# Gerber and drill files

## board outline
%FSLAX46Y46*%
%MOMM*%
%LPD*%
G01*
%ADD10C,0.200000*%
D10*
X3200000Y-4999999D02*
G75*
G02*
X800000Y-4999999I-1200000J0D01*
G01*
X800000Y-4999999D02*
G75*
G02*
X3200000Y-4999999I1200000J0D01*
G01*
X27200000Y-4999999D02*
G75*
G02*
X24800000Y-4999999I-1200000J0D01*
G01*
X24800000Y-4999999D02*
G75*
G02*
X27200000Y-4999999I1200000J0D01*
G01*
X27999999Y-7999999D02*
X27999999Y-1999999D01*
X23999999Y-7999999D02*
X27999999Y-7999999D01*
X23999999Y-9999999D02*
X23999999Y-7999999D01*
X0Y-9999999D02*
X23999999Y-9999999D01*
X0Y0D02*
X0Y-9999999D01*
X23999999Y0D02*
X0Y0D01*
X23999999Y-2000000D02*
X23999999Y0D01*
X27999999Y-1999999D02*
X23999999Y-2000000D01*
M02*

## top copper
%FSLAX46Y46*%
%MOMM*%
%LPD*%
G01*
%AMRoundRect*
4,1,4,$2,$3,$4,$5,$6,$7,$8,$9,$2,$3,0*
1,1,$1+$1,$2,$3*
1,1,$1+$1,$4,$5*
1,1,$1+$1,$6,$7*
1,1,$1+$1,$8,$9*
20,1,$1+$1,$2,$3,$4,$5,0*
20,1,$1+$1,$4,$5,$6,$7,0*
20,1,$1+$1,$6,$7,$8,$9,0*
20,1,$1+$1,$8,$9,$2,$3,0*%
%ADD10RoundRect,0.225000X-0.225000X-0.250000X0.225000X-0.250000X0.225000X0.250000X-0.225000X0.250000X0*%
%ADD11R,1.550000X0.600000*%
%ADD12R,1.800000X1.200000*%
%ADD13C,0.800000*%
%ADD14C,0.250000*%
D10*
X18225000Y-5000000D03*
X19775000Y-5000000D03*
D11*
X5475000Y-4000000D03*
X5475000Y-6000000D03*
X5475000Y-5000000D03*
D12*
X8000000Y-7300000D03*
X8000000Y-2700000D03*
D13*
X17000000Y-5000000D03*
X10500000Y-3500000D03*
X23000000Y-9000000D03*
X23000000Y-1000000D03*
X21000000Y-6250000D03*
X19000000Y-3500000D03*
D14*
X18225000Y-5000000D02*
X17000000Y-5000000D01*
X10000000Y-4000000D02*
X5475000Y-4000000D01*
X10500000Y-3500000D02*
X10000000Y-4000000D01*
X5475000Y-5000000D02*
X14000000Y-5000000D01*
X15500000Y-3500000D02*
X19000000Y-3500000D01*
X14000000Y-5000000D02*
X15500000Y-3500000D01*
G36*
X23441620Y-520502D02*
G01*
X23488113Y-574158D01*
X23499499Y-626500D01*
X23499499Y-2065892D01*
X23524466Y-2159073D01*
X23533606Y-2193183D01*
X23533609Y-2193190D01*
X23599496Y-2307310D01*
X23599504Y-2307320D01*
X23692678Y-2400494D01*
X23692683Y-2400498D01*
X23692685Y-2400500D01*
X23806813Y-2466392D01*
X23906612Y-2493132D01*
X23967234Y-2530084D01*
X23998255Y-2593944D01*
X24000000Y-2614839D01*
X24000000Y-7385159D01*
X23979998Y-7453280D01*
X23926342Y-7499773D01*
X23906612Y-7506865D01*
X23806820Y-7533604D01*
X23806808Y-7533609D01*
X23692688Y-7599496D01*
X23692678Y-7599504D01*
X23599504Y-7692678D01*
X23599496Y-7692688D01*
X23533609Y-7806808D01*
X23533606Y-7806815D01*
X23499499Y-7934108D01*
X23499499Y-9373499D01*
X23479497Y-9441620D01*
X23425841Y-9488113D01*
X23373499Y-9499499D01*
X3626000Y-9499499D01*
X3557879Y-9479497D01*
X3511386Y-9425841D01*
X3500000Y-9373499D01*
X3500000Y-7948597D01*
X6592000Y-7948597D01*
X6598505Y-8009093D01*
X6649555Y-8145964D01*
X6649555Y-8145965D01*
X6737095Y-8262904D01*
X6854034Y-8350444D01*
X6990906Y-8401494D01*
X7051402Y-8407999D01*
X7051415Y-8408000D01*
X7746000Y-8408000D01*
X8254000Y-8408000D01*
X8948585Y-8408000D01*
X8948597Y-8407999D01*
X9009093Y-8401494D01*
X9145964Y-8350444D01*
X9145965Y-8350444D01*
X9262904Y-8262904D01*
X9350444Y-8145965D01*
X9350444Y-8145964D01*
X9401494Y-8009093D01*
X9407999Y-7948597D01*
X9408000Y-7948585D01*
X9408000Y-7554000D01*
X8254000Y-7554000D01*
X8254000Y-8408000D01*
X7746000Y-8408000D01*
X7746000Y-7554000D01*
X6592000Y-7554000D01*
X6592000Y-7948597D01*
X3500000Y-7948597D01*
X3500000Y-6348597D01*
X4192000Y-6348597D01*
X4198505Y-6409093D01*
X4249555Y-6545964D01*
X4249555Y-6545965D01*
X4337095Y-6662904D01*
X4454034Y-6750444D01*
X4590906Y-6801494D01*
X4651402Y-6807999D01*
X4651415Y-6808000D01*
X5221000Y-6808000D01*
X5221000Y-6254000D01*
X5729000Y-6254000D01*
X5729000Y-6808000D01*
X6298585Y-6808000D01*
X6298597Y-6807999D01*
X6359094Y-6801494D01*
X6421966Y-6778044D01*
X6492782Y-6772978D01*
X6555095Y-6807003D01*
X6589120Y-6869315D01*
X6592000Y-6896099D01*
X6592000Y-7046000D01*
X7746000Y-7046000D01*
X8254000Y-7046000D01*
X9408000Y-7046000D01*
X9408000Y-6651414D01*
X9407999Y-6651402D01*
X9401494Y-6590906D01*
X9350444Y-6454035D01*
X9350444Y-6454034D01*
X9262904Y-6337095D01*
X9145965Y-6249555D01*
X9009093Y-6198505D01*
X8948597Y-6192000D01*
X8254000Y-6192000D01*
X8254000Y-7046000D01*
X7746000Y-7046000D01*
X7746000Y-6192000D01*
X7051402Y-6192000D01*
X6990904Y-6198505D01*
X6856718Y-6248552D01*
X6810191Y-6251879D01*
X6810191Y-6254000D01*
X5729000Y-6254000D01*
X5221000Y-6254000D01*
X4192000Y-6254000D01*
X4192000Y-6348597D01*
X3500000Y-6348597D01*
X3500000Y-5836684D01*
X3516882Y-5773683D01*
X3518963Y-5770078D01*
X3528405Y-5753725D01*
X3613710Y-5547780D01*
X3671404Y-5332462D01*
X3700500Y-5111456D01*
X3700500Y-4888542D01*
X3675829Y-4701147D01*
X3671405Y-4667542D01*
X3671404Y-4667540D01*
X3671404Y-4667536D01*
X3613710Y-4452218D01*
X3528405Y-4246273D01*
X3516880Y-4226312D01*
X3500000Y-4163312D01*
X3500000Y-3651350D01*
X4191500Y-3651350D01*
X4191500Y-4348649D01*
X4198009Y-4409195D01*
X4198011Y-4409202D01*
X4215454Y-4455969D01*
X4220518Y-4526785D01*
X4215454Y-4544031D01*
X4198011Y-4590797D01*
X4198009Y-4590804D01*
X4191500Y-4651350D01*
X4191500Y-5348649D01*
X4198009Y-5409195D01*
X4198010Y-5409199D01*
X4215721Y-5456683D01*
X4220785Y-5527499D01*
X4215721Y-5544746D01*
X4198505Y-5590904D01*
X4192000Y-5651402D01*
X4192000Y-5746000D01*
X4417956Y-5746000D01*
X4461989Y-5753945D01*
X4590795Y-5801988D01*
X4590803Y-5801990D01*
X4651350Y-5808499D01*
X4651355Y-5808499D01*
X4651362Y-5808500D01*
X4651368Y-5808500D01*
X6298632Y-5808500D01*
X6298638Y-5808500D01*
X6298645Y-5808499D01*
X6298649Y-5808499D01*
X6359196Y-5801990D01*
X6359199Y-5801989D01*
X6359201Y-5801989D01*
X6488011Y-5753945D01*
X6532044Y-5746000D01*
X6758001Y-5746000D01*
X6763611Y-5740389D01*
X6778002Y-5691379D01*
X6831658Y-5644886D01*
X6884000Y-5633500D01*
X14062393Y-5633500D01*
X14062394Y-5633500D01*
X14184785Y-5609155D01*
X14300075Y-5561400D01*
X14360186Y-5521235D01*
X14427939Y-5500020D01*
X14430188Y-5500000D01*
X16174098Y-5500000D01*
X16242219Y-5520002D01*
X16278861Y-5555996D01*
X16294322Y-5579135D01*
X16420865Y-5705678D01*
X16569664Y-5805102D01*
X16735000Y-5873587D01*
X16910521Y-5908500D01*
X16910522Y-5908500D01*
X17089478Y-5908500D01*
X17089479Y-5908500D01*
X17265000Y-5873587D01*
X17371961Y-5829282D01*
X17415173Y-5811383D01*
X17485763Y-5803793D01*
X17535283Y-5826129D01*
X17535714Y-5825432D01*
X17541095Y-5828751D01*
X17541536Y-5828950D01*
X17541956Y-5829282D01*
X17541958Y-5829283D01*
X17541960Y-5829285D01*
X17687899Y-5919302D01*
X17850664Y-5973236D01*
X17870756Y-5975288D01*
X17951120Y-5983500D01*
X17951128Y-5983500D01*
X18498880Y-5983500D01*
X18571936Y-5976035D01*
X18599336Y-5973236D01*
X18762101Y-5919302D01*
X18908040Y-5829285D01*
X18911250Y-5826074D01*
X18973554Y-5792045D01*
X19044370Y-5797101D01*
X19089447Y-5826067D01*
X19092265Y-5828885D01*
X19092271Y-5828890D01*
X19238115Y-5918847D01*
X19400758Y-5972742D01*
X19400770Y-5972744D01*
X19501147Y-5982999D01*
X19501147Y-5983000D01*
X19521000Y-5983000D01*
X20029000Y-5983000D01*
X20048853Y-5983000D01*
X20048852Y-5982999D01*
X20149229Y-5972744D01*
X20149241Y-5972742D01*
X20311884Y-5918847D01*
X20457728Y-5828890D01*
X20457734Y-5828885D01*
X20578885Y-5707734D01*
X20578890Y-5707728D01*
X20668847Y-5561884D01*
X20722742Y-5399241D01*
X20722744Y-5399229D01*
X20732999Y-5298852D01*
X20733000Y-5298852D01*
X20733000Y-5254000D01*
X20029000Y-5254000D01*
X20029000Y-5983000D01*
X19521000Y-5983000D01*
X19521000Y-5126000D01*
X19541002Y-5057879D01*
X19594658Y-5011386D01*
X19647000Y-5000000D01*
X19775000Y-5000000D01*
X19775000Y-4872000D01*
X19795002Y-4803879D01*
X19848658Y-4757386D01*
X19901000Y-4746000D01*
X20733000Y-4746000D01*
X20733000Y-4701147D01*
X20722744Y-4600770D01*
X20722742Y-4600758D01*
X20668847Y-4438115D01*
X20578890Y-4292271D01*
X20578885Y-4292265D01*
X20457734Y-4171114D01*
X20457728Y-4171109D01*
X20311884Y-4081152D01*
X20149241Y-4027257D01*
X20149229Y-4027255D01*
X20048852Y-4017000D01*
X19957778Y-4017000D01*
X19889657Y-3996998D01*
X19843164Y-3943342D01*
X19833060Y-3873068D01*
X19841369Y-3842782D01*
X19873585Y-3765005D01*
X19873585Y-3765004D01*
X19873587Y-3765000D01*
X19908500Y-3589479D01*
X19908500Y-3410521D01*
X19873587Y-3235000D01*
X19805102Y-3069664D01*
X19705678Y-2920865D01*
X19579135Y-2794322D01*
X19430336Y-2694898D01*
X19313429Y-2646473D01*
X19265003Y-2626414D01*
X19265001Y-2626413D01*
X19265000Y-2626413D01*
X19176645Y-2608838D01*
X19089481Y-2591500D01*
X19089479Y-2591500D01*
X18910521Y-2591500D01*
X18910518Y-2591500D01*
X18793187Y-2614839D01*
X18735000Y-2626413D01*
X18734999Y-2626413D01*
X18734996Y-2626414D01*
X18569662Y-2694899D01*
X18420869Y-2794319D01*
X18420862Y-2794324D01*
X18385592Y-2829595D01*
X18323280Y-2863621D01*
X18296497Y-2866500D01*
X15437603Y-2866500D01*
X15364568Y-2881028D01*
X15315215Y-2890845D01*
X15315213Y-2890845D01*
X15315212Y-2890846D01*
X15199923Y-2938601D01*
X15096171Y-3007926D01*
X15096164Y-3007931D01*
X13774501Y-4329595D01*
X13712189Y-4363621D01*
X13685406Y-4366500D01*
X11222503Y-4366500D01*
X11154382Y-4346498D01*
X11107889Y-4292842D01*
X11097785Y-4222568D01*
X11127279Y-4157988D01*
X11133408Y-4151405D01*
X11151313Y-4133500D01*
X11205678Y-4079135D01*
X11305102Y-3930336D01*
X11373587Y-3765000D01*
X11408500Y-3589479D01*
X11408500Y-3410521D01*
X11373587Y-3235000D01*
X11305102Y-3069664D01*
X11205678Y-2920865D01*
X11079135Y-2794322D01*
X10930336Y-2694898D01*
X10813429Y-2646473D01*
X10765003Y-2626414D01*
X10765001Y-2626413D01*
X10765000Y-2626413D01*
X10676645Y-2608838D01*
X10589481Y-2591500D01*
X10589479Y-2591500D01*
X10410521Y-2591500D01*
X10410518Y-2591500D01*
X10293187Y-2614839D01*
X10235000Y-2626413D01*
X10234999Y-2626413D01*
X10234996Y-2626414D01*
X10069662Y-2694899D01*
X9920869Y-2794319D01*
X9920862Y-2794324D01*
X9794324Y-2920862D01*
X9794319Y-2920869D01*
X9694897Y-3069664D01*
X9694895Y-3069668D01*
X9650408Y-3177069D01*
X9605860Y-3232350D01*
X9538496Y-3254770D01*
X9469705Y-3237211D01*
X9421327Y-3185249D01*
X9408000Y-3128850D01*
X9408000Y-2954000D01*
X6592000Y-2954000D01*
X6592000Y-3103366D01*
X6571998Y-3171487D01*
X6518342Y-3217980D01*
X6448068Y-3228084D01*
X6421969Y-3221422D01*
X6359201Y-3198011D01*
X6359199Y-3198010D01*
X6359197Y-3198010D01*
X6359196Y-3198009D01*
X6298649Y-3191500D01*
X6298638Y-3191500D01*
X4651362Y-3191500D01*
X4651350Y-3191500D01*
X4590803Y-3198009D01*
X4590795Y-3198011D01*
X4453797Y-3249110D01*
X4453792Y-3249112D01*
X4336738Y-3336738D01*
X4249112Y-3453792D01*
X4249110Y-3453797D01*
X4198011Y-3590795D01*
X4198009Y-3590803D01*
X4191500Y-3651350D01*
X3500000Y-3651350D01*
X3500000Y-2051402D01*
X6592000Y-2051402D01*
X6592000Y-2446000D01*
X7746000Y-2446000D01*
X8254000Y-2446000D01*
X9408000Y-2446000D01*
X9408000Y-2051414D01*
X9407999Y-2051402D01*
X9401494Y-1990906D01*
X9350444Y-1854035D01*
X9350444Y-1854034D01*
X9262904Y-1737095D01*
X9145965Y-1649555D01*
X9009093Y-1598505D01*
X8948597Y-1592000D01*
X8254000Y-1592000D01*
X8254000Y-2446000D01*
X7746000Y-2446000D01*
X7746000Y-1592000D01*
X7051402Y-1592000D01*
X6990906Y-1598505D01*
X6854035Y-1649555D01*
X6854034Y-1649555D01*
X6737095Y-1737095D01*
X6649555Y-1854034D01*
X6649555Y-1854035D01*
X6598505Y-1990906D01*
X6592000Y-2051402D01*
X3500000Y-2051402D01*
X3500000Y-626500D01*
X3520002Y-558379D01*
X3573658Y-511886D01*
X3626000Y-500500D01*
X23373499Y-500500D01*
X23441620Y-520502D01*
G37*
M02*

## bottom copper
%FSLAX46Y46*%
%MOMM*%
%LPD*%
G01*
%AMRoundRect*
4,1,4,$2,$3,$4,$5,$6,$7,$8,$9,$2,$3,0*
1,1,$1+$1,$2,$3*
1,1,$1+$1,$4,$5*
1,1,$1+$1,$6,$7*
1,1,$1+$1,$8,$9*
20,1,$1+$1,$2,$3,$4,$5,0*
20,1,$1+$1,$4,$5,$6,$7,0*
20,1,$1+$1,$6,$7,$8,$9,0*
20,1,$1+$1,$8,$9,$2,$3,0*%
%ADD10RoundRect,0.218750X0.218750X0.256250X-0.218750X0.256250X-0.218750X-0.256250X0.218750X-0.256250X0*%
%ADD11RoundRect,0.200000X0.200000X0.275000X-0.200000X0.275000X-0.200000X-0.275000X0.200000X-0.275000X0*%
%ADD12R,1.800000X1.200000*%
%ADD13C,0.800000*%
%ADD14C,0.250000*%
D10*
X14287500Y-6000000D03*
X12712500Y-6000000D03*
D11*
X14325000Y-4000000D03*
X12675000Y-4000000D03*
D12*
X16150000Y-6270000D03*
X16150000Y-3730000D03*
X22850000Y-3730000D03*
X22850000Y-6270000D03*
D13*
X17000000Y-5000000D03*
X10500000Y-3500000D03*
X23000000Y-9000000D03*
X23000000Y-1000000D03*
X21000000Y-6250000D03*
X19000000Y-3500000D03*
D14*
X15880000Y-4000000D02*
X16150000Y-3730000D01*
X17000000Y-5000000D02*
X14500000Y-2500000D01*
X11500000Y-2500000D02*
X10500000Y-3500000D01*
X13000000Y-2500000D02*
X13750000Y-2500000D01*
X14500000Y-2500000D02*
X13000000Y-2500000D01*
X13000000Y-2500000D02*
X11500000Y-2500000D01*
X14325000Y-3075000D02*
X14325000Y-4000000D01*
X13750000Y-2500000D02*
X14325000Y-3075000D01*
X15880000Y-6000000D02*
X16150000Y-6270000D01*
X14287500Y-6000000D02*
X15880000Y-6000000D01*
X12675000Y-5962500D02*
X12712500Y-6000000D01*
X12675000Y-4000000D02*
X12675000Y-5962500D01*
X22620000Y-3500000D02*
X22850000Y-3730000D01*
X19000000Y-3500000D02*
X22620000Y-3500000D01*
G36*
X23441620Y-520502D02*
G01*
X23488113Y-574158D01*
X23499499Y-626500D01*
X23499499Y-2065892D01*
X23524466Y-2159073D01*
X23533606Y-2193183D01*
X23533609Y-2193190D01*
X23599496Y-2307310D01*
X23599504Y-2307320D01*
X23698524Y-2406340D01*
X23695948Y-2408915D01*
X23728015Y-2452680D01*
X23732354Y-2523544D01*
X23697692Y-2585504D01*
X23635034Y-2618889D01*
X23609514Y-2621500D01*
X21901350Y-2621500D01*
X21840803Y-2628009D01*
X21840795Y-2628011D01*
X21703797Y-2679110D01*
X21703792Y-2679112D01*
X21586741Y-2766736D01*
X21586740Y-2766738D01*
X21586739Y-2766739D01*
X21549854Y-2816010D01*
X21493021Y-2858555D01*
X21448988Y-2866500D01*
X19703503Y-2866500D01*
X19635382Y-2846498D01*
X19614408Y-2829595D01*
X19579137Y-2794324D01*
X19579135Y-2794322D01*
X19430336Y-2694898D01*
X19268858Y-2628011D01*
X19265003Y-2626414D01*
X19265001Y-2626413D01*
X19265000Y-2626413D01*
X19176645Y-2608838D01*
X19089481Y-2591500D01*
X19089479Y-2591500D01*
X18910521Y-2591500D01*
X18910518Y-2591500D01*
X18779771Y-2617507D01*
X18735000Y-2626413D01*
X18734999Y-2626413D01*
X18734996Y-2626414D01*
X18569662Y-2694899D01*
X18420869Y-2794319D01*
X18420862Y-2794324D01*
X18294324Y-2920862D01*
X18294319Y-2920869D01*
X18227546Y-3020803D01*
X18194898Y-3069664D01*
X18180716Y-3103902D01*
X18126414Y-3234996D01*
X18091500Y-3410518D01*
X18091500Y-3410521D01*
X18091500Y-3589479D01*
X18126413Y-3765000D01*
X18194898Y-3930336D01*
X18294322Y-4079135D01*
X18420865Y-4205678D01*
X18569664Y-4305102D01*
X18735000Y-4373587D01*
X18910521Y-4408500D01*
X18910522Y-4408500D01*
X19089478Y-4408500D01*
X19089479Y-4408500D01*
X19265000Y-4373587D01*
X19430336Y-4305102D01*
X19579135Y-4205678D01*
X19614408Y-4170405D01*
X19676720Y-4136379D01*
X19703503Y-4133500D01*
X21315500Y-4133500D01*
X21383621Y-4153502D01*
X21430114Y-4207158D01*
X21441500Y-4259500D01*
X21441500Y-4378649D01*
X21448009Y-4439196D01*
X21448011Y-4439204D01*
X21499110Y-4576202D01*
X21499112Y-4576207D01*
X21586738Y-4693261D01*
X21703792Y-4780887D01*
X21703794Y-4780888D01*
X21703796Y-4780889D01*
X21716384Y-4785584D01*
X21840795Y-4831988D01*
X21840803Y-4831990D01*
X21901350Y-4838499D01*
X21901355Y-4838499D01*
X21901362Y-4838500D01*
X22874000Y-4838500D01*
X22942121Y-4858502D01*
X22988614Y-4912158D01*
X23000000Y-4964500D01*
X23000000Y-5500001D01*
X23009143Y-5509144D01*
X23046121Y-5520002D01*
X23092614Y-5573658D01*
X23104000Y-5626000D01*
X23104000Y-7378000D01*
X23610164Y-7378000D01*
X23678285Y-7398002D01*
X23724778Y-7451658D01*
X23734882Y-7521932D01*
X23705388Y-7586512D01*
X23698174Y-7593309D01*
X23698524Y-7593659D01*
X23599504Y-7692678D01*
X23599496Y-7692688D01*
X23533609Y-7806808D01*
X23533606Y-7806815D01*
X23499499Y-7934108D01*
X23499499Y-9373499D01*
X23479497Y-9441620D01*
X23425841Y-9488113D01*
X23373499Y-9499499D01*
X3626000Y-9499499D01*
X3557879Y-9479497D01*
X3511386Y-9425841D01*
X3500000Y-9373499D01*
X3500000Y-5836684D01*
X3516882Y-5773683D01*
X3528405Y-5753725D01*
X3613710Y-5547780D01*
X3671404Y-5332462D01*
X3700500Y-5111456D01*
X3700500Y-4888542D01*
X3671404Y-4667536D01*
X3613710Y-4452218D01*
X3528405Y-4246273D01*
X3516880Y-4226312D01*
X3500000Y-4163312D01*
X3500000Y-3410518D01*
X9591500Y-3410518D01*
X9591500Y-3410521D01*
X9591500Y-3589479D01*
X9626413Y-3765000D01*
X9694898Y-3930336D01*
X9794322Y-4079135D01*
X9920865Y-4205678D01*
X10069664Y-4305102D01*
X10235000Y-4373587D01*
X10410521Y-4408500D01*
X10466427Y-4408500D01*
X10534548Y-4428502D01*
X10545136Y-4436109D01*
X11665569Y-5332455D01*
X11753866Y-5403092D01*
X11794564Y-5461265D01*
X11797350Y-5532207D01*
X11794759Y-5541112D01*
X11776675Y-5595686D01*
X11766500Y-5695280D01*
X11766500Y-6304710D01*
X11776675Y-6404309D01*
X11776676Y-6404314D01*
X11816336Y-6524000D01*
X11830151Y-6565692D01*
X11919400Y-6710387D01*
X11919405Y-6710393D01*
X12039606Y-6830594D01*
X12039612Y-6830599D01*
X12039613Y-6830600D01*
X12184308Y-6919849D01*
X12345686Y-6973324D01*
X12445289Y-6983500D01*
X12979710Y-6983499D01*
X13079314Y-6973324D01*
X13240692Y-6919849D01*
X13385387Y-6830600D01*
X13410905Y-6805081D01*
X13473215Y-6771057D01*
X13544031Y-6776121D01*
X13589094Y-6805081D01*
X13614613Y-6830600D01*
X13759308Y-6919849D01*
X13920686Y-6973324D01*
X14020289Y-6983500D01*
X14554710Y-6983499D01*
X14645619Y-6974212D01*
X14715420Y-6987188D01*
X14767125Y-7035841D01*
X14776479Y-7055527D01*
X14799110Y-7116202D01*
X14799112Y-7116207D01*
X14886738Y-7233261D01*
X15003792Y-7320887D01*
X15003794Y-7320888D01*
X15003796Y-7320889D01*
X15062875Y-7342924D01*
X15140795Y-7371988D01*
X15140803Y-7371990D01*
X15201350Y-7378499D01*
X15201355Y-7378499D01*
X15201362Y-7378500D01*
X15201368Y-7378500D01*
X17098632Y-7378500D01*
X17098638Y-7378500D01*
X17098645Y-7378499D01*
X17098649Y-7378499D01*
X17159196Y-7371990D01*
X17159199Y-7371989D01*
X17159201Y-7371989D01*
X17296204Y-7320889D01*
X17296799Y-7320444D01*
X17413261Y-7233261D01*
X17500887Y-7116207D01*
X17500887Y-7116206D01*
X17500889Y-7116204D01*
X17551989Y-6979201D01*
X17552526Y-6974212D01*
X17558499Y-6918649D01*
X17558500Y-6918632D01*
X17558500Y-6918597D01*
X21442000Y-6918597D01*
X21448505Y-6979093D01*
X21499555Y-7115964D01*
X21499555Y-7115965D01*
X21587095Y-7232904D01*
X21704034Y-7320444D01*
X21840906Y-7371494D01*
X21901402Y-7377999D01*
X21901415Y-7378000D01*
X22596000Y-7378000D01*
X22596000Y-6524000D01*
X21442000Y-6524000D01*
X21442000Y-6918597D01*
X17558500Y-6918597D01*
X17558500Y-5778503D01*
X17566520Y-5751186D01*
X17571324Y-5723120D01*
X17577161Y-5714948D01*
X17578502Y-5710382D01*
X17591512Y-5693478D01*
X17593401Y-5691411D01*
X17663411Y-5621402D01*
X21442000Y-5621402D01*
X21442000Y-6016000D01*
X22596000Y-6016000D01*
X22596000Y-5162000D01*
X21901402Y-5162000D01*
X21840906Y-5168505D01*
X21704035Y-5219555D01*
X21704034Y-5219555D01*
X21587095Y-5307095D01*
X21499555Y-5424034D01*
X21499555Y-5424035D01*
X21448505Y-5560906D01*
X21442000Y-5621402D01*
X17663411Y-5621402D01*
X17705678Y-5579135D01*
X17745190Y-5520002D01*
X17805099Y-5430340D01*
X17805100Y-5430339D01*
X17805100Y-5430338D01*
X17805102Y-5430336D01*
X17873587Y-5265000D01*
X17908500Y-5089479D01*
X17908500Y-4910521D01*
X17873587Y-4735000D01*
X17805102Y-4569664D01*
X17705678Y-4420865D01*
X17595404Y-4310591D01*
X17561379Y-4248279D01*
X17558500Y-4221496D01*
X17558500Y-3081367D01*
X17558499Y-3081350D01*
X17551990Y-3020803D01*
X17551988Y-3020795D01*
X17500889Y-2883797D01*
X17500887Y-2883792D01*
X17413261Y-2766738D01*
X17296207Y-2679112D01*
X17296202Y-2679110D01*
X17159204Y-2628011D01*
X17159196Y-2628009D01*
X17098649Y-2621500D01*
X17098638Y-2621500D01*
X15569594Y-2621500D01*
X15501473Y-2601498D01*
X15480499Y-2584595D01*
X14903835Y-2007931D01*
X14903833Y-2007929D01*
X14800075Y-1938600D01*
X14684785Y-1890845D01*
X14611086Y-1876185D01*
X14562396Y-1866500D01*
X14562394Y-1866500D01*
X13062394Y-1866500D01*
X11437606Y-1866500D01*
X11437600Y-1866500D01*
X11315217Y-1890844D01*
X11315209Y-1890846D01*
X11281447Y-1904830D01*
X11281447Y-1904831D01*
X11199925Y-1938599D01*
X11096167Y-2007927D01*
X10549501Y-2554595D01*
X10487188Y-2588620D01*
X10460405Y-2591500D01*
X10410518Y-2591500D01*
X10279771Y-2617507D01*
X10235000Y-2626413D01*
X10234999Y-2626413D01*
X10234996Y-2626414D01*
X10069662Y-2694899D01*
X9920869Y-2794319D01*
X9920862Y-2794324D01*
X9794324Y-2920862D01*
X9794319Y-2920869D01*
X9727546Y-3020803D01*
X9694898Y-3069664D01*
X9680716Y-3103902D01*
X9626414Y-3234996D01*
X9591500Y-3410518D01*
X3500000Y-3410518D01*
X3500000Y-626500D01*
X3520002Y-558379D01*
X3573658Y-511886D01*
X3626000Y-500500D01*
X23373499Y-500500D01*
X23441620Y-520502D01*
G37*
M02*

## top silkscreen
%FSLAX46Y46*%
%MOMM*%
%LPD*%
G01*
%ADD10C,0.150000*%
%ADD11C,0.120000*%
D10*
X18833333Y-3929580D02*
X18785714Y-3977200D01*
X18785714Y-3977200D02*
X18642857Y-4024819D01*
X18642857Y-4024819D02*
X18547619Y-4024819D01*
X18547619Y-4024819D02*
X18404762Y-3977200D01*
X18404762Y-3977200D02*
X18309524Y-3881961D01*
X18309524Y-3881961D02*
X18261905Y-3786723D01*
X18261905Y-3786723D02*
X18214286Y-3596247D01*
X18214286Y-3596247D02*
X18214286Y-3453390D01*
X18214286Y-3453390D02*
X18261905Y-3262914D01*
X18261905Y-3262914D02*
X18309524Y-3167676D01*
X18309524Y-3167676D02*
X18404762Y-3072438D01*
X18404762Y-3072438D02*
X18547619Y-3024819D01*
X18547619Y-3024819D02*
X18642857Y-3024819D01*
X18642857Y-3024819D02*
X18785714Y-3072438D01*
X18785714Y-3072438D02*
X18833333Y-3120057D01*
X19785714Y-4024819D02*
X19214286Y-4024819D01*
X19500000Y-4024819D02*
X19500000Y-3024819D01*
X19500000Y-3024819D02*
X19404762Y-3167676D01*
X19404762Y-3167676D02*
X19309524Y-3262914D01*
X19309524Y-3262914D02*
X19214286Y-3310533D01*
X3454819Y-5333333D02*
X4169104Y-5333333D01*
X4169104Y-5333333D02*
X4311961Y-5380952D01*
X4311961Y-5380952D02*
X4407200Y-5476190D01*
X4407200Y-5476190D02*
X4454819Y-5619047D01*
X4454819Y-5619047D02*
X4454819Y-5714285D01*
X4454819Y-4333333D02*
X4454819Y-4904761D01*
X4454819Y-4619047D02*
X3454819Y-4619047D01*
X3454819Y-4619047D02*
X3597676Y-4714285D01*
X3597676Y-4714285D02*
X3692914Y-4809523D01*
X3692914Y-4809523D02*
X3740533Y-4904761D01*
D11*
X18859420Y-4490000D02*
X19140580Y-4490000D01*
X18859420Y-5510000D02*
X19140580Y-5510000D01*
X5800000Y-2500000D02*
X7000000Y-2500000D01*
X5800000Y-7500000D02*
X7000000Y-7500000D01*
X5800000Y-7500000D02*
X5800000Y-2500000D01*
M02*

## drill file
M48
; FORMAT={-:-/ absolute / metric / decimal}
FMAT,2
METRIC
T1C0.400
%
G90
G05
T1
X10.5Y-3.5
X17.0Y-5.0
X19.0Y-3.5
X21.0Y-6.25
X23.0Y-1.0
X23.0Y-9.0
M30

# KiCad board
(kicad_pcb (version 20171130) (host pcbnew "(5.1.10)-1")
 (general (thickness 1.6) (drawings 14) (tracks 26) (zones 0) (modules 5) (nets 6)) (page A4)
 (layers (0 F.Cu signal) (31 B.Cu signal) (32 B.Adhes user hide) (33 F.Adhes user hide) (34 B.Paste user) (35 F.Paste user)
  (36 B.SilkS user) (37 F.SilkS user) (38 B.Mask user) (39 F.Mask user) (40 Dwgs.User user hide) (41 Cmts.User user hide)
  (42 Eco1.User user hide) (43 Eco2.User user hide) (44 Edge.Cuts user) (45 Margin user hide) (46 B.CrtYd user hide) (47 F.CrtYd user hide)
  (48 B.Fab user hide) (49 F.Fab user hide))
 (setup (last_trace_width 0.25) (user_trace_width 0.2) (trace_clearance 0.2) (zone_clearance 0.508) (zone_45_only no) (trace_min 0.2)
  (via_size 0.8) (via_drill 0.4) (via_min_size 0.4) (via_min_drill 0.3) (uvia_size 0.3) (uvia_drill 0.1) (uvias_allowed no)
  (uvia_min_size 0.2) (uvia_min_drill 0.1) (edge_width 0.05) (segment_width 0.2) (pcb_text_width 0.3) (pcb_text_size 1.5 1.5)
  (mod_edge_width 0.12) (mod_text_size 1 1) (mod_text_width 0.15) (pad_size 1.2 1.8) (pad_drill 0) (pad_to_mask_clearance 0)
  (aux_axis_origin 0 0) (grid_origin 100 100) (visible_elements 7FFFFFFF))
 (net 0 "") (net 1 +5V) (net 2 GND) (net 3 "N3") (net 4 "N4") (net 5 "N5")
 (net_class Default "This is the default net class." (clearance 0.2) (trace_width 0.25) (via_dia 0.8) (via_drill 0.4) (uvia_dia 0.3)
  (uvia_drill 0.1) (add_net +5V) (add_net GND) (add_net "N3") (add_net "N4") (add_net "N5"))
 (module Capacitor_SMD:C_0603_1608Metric (layer F.Cu) (at 19 5)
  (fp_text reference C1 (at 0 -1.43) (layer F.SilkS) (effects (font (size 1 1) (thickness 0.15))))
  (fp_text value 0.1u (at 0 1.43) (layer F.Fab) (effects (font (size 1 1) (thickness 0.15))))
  (fp_line (start -0.14058 -0.51) (end 0.14058 -0.51) (layer F.SilkS) (width 0.12))
  (fp_line (start -0.14058 0.51) (end 0.14058 0.51) (layer F.SilkS) (width 0.12))
  (pad 1 smd roundrect (at -0.775 0) (size 0.9 0.95) (layers F.Cu F.Paste F.Mask) (roundrect_rratio 0.25) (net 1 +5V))
  (pad 2 smd roundrect (at 0.775 0) (size 0.9 0.95) (layers F.Cu F.Paste F.Mask) (roundrect_rratio 0.25) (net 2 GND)))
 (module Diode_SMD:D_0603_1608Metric (layer B.Cu) (at 13.5 6 180)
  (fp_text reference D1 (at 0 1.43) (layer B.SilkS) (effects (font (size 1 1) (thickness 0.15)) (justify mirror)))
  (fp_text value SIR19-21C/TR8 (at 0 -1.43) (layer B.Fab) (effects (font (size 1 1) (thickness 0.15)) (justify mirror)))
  (pad 1 smd roundrect (at -0.7875 0 180) (size 0.875 0.95) (layers B.Cu B.Paste B.Mask) (roundrect_rratio 0.25) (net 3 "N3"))
  (pad 2 smd roundrect (at 0.7875 0 180) (size 0.875 0.95) (layers B.Cu B.Paste B.Mask) (roundrect_rratio 0.25) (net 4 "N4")))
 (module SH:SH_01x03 (layer F.Cu) (at 8 5 90)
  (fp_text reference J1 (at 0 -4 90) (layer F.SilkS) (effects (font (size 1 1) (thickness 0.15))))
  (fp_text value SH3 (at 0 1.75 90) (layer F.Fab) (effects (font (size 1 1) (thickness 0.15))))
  (fp_line (start 2.5 -2.2) (end 2.5 -1) (layer F.SilkS) (width 0.12))
  (fp_line (start -2.5 -2.2) (end -2.5 -1) (layer F.SilkS) (width 0.12))
  (fp_line (start -2.5 -2.2) (end 2.5 -2.2) (layer F.SilkS) (width 0.12))
  (pad 3 smd rect (at 1 -2.525 90) (size 0.6 1.55) (layers F.Cu F.Paste F.Mask) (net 1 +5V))
  (pad 1 smd rect (at -1 -2.525 90) (size 0.6 1.55) (layers F.Cu F.Paste F.Mask) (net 2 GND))
  (pad 2 smd rect (at 0 -2.525 90) (size 0.6 1.55) (layers F.Cu F.Paste F.Mask) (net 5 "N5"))
  (pad MP smd rect (at -2.3 0 90) (size 1.2 1.8) (layers F.Cu F.Paste F.Mask) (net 2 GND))
  (pad MP smd rect (at 2.3 0 90) (size 1.2 1.8) (layers F.Cu F.Paste F.Mask) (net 2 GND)))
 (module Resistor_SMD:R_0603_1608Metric (layer B.Cu) (at 13.5 4 180)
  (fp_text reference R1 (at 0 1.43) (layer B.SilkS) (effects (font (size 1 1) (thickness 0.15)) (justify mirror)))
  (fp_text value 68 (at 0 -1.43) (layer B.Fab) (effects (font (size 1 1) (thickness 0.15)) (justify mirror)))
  (pad 1 smd roundrect (at -0.825 0 180) (size 0.8 0.95) (layers B.Cu B.Paste B.Mask) (roundrect_rratio 0.25) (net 1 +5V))
  (pad 2 smd roundrect (at 0.825 0 180) (size 0.8 0.95) (layers B.Cu B.Paste B.Mask) (roundrect_rratio 0.25) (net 4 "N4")))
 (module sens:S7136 (layer B.Cu) (at 19.5 5)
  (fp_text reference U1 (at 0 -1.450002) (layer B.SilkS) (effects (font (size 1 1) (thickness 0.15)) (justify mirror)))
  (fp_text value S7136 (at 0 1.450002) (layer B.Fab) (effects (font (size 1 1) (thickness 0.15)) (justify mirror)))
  (pad 1 smd rect (at -3.35 1.27) (size 1.8 1.2) (layers B.Cu B.Paste B.Mask) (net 3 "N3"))
  (pad 2 smd rect (at -3.35 -1.27) (size 1.8 1.2) (layers B.Cu B.Paste B.Mask) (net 1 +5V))
  (pad 3 smd rect (at 3.35 -1.27) (size 1.8 1.2) (layers B.Cu B.Paste B.Mask) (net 5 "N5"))
  (pad 4 smd rect (at 3.35 1.27) (size 1.8 1.2) (layers B.Cu B.Paste B.Mask) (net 2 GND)))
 (gr_circle (center 2 4.999999) (end 3.2 4.999999) (layer Edge.Cuts) (width 0.2))
 (gr_circle (center 26 4.999999) (end 27.2 4.999999) (layer Edge.Cuts) (width 0.2))
 (gr_line (start 27.999999 7.999999) (end 27.999999 1.999999) (layer Edge.Cuts) (width 0.2))
 (gr_line (start 23.999999 7.999999) (end 27.999999 7.999999) (layer Edge.Cuts) (width 0.2))
 (gr_line (start 23.999999 9.999999) (end 23.999999 7.999999) (layer Edge.Cuts) (width 0.2))
 (gr_line (start 0 9.999999) (end 23.999999 9.999999) (layer Edge.Cuts) (width 0.2))
 (gr_line (start 0 0) (end 0 9.999999) (layer Edge.Cuts) (width 0.2))
 (gr_line (start 23.999999 0) (end 0 0) (layer Edge.Cuts) (width 0.2))
 (gr_line (start 23.999999 2) (end 23.999999 0) (layer Edge.Cuts) (width 0.2))
 (gr_line (start 27.999999 1.999999) (end 23.999999 2) (layer Edge.Cuts) (width 0.2))
 (segment (start 15.88 4) (end 16.15 3.73) (width 0.25) (layer B.Cu) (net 1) (status 30))
 (via (at 17 5) (size 0.8) (drill 0.4) (layers F.Cu B.Cu) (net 1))
 (segment (start 18.225 5) (end 17 5) (width 0.25) (layer F.Cu) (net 1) (status 10))
 (segment (start 17 5) (end 14.5 2.5) (width 0.25) (layer B.Cu) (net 1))
 (via (at 10.5 3.5) (size 0.8) (drill 0.4) (layers F.Cu B.Cu) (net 1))
 (segment (start 11.5 2.5) (end 10.5 3.5) (width 0.25) (layer B.Cu) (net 1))
 (segment (start 10 4) (end 5.475 4) (width 0.25) (layer F.Cu) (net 1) (status 20))
 (segment (start 10.5 3.5) (end 10 4) (width 0.25) (layer F.Cu) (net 1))
 (segment (start 13 2.5) (end 13.75 2.5) (width 0.25) (layer B.Cu) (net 1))
 (segment (start 14.5 2.5) (end 13 2.5) (width 0.25) (layer B.Cu) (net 1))
 (segment (start 13 2.5) (end 11.5 2.5) (width 0.25) (layer B.Cu) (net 1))
 (segment (start 14.325 3.075) (end 14.325 4) (width 0.25) (layer B.Cu) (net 1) (status 20))
 (segment (start 13.75 2.5) (end 14.325 3.075) (width 0.25) (layer B.Cu) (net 1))
 (via (at 23 9) (size 0.8) (drill 0.4) (layers F.Cu B.Cu) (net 2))
 (via (at 23 1) (size 0.8) (drill 0.4) (layers F.Cu B.Cu) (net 2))
 (via (at 21 6.25) (size 0.8) (drill 0.4) (layers F.Cu B.Cu) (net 2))
 (segment (start 15.88 6) (end 16.15 6.27) (width 0.25) (layer B.Cu) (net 3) (status 30))
 (segment (start 14.2875 6) (end 15.88 6) (width 0.25) (layer B.Cu) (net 3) (status 30))
 (segment (start 12.675 5.9625) (end 12.7125 6) (width 0.25) (layer B.Cu) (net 4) (status 30))
 (segment (start 12.675 4) (end 12.675 5.9625) (width 0.25) (layer B.Cu) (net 4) (status 30))
 (segment (start 5.475 5) (end 14 5) (width 0.25) (layer F.Cu) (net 5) (status 10))
 (via (at 19 3.5) (size 0.8) (drill 0.4) (layers F.Cu B.Cu) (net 5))
 (segment (start 15.5 3.5) (end 19 3.5) (width 0.25) (layer F.Cu) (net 5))
 (segment (start 14 5) (end 15.5 3.5) (width 0.25) (layer F.Cu) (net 5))
 (segment (start 22.62 3.5) (end 22.85 3.73) (width 0.25) (layer B.Cu) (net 5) (status 30))
 (segment (start 19 3.5) (end 22.62 3.5) (width 0.25) (layer B.Cu) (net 5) (status 20))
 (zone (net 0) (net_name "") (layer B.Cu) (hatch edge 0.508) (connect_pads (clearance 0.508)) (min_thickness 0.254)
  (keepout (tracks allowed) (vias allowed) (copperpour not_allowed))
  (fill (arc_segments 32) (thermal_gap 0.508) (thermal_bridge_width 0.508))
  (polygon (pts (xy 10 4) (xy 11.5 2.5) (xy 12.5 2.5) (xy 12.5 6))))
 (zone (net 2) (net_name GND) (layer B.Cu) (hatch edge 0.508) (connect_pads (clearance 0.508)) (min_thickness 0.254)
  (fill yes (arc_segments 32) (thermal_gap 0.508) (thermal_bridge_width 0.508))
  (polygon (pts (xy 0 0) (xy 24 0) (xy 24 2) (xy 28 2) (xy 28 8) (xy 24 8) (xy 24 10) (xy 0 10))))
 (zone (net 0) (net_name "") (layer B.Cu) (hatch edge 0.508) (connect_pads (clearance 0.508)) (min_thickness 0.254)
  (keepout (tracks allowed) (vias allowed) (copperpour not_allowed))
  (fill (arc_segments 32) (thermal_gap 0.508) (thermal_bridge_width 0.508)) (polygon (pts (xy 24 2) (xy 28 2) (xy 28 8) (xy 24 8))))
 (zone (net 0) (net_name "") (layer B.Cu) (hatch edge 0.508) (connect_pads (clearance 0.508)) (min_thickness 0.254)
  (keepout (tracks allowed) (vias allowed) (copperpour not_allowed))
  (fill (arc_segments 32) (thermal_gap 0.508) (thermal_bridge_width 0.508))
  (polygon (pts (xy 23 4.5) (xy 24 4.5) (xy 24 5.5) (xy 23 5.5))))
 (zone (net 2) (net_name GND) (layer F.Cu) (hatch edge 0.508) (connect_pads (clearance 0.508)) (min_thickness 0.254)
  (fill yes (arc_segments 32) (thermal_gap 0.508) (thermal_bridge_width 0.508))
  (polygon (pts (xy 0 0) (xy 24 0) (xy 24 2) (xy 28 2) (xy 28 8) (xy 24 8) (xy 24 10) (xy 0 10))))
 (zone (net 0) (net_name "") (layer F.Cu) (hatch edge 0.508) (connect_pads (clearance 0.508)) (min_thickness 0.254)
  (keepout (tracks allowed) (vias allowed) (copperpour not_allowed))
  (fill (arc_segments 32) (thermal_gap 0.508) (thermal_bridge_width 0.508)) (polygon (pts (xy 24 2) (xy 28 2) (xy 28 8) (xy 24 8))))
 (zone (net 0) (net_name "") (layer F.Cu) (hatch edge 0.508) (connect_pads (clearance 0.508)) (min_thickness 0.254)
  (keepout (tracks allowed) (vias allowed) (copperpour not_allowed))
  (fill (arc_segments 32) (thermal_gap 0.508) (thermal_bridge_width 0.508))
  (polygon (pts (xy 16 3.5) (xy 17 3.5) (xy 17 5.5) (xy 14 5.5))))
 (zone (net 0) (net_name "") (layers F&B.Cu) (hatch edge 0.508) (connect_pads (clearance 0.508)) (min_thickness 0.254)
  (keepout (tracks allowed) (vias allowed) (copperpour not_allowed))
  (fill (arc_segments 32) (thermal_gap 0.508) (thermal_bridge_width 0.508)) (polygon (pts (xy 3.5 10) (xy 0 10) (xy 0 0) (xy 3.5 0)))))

